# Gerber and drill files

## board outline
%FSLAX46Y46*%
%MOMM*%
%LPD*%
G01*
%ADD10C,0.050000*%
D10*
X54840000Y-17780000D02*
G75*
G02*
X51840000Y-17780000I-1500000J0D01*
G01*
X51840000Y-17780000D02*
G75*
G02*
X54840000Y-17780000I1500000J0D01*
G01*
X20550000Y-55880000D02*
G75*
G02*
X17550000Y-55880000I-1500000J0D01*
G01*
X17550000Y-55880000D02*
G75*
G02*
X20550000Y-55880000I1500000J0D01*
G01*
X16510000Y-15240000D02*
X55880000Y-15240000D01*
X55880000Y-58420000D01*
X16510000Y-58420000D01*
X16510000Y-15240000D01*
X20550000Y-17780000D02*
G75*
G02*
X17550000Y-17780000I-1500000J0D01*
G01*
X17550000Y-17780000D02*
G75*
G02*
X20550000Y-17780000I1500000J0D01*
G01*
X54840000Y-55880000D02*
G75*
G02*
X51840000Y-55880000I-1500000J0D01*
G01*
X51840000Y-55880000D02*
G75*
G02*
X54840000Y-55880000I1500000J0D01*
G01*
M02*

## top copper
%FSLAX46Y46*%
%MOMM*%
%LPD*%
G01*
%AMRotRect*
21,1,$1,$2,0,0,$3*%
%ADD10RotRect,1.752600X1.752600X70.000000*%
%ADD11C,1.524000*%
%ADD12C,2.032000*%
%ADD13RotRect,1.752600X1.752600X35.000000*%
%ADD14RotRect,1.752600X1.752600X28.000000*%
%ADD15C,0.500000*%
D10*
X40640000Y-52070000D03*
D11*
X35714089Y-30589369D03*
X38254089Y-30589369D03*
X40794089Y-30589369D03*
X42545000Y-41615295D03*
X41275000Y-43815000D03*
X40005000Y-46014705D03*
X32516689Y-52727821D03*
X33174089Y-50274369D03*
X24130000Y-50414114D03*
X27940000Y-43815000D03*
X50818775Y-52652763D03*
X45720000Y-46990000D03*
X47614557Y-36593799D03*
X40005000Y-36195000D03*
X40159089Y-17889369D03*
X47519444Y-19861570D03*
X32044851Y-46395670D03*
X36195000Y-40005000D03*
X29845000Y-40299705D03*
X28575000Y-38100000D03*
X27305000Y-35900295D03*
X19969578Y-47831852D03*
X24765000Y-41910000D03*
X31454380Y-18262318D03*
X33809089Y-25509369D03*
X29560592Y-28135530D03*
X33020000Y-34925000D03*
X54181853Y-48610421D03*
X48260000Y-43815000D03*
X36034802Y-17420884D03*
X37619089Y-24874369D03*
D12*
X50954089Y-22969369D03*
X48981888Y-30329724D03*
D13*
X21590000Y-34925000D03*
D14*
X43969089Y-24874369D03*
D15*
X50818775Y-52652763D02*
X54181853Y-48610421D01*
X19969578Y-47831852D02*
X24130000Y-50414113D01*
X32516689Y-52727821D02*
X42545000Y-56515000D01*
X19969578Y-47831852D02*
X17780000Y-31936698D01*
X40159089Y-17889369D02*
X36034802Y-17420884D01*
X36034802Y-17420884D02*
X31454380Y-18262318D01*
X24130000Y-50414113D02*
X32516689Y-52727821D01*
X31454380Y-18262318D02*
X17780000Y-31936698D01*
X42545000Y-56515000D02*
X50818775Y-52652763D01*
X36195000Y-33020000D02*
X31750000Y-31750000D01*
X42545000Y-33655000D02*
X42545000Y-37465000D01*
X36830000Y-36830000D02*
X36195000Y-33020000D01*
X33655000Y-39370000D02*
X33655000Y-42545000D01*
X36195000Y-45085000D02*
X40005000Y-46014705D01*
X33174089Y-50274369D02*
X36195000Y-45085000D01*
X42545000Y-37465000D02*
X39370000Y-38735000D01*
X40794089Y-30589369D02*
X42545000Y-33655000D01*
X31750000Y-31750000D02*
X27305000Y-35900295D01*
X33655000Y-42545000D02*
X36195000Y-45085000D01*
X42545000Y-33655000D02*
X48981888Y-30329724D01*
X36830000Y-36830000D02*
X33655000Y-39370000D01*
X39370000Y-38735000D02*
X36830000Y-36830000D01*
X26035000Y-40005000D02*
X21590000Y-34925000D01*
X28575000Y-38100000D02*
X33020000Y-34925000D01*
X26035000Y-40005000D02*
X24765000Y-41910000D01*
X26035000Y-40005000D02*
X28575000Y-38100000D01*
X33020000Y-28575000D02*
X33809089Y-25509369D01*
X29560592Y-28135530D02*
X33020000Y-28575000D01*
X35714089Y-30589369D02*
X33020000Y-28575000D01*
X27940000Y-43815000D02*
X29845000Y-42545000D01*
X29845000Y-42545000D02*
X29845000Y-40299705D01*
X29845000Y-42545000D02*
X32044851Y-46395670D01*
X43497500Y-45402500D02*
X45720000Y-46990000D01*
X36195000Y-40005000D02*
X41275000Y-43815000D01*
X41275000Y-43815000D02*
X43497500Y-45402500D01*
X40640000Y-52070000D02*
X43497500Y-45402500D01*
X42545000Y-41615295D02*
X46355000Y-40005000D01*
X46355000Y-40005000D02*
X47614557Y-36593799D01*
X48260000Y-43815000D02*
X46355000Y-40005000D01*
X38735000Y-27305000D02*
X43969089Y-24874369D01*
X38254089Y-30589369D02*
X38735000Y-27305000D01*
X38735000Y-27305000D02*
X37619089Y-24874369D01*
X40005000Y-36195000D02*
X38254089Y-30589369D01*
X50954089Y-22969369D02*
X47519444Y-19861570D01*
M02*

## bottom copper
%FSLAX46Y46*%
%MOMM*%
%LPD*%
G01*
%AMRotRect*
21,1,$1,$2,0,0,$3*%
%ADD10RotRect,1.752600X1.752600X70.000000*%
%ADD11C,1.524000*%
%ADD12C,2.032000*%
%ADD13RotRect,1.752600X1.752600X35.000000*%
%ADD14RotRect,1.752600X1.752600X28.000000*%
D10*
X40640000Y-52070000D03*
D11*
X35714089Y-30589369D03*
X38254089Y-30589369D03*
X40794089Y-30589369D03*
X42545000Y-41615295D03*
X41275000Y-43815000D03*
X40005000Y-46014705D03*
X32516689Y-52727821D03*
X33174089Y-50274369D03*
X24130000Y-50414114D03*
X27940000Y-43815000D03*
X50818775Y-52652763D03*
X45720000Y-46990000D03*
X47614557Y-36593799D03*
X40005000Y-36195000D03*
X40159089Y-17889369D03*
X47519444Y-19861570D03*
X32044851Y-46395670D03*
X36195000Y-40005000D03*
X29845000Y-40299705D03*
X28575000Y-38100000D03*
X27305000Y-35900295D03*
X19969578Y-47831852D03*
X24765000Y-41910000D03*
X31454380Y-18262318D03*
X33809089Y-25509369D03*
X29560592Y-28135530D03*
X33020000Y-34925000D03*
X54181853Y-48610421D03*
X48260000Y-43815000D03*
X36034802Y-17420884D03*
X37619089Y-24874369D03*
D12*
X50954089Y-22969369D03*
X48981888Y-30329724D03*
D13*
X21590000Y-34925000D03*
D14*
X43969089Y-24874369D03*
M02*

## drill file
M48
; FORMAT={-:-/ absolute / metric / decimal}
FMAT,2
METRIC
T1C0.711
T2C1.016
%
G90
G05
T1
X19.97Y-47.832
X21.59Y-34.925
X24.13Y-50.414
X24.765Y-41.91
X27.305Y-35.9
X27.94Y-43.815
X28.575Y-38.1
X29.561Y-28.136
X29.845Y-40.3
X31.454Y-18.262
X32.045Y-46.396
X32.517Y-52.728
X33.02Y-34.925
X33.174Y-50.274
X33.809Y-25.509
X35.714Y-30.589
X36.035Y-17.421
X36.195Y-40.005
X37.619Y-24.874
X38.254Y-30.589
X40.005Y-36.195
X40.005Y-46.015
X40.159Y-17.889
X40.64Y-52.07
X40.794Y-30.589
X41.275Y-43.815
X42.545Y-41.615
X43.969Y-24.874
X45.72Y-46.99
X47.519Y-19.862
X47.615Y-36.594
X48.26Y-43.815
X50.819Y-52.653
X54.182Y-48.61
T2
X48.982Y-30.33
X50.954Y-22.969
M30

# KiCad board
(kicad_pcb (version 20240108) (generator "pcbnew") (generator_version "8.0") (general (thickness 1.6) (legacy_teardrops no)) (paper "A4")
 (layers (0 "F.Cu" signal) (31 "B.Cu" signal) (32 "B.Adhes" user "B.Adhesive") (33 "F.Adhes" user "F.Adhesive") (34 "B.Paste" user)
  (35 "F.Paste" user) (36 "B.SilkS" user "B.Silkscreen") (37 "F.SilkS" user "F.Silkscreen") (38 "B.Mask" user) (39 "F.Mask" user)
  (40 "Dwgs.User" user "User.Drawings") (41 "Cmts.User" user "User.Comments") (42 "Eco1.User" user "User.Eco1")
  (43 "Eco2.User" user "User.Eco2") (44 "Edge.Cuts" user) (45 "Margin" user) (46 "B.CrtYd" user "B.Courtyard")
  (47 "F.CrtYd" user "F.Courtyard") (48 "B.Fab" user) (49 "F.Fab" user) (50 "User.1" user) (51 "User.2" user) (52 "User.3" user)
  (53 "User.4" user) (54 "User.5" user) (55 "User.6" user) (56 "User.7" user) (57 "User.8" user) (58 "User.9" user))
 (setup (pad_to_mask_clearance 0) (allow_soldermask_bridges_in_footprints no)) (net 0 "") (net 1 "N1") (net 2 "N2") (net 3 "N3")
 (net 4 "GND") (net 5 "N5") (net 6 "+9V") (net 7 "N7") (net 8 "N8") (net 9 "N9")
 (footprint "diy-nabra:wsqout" (layer "F.Cu") (at 40.64 52.07 70)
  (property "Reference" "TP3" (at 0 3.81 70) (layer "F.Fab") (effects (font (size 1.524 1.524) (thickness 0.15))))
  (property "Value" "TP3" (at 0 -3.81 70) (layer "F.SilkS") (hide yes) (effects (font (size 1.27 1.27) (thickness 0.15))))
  (pad "1" thru_hole rect (at 0 0 70) (size 1.7526 1.7526) (drill 0.7112) (layers "*.Cu" "*.Mask") (remove_unused_layers no) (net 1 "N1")))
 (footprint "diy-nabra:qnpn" (layer "F.Cu") (at 38.254089 30.589369 180)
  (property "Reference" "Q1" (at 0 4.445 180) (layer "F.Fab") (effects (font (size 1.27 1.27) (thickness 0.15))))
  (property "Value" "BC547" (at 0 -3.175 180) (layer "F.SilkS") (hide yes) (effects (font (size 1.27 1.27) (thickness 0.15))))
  (pad "1" thru_hole circle (at 2.54 0 180) (size 1.524 1.524) (drill 0.7112) (layers "*.Cu" "*.Mask") (remove_unused_layers no)
   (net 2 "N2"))
  (pad "2" thru_hole circle (at 0 0 180) (size 1.524 1.524) (drill 0.7112) (layers "*.Cu" "*.Mask") (remove_unused_layers no) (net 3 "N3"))
  (pad "3" thru_hole circle (at -2.54 0 180) (size 1.524 1.524) (drill 0.7112) (layers "*.Cu" "*.Mask") (remove_unused_layers no)
   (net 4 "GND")))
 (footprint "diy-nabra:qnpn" (layer "F.Cu") (at 41.275 43.815 60)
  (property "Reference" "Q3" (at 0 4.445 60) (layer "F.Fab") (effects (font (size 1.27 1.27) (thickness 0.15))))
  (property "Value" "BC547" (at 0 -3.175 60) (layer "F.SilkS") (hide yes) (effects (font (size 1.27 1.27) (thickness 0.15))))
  (pad "1" thru_hole circle (at 2.54 0 60) (size 1.524 1.524) (drill 0.7112) (layers "*.Cu" "*.Mask") (remove_unused_layers no) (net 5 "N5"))
  (pad "2" thru_hole circle (at 0 0 60) (size 1.524 1.524) (drill 0.7112) (layers "*.Cu" "*.Mask") (remove_unused_layers no) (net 1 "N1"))
  (pad "3" thru_hole circle (at -2.54 0 60) (size 1.524 1.524) (drill 0.7112) (layers "*.Cu" "*.Mask") (remove_unused_layers no)
   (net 4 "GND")))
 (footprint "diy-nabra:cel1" (layer "F.Cu") (at 33.174089 50.274369 -105)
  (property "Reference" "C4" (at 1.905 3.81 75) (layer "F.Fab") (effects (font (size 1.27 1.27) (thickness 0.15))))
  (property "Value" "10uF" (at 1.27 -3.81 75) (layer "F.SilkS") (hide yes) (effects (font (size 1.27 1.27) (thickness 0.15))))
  (pad "1" thru_hole circle (at 2.54 0 255) (size 1.524 1.524) (drill 0.7112) (layers "*.Cu" "*.Mask") (remove_unused_layers no)
   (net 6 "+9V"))
  (pad "2" thru_hole circle (at 0 0 255) (size 1.524 1.524) (drill 0.7112) (layers "*.Cu" "*.Mask") (remove_unused_layers no) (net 4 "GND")))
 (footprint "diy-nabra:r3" (layer "F.Cu") (at 27.94 43.815 -120)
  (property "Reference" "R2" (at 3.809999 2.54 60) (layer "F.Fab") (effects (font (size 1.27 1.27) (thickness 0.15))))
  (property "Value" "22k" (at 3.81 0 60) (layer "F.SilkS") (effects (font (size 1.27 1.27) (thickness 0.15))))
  (pad "1" thru_hole circle (at 7.62 0 240) (size 1.524 1.524) (drill 0.7112) (layers "*.Cu" "*.Mask") (remove_unused_layers no)
   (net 6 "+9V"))
  (pad "2" thru_hole circle (at 0 0 240) (size 1.524 1.524) (drill 0.7112) (layers "*.Cu" "*.Mask") (remove_unused_layers no) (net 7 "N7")))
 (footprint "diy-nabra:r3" (layer "F.Cu") (at 45.72 46.99 -48)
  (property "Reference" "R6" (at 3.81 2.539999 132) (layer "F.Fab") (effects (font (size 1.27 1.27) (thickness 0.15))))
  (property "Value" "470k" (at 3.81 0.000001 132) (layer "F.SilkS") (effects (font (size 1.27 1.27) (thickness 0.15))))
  (pad "1" thru_hole circle (at 7.619999 0 312) (size 1.524 1.524) (drill 0.7112) (layers "*.Cu" "*.Mask") (remove_unused_layers no)
   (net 6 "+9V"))
  (pad "2" thru_hole circle (at 0 0 312) (size 1.524 1.524) (drill 0.7112) (layers "*.Cu" "*.Mask") (remove_unused_layers no) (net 1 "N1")))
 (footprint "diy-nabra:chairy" (layer "F.Cu") (at 40.005 36.195 -3)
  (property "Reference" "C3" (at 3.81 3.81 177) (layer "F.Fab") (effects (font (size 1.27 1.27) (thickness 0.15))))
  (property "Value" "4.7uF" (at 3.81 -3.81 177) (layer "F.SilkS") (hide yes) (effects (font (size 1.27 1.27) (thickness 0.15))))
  (pad "1" thru_hole circle (at 7.62 -0.000001 357) (size 1.524 1.524) (drill 0.7112) (layers "*.Cu" "*.Mask") (remove_unused_layers no)
   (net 5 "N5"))
  (pad "2" thru_hole circle (at 0 0 357) (size 1.524 1.524) (drill 0.7112) (layers "*.Cu" "*.Mask") (remove_unused_layers no) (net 3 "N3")))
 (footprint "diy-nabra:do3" (layer "F.Cu") (at 40.159089 17.889369 -15)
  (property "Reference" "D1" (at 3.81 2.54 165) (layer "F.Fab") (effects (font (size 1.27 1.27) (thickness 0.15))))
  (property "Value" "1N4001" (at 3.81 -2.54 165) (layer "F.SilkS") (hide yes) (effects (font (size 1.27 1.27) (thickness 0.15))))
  (pad "1" thru_hole circle (at 0 0 345) (size 1.524 1.524) (drill 0.7112) (layers "*.Cu" "*.Mask") (remove_unused_layers no) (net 6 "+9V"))
  (pad "2" thru_hole circle (at 7.62 0 345) (size 1.524 1.524) (drill 0.7112) (layers "*.Cu" "*.Mask") (remove_unused_layers no)
   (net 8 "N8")))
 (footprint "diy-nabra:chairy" (layer "F.Cu") (at 36.195 40.005 -123)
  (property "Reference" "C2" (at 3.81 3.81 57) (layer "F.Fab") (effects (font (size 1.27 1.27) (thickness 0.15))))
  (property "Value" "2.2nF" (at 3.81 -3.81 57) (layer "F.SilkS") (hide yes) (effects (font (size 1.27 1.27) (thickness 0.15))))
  (pad "1" thru_hole circle (at 7.62 -0.000001 237) (size 1.524 1.524) (drill 0.7112) (layers "*.Cu" "*.Mask") (remove_unused_layers no)
   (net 7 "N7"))
  (pad "2" thru_hole circle (at 0 0 237) (size 1.524 1.524) (drill 0.7112) (layers "*.Cu" "*.Mask") (remove_unused_layers no) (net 1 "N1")))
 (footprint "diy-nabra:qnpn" (layer "F.Cu") (at 28.575 38.1 -60)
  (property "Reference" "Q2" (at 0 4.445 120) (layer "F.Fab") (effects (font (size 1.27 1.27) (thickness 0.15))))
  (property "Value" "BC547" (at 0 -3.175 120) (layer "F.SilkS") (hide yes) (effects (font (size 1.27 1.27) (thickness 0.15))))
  (pad "1" thru_hole circle (at 2.54 0 300) (size 1.524 1.524) (drill 0.7112) (layers "*.Cu" "*.Mask") (remove_unused_layers no)
   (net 7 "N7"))
  (pad "2" thru_hole circle (at 0 0 300) (size 1.524 1.524) (drill 0.7112) (layers "*.Cu" "*.Mask") (remove_unused_layers no) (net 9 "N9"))
  (pad "3" thru_hole circle (at -2.54 0 300) (size 1.524 1.524) (drill 0.7112) (layers "*.Cu" "*.Mask") (remove_unused_layers no)
   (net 4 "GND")))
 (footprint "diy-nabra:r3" (layer "F.Cu") (at 24.765 41.91 -129)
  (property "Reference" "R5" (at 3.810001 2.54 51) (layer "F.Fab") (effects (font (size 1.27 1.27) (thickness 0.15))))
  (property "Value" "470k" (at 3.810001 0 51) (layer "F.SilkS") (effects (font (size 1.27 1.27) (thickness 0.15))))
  (pad "1" thru_hole circle (at 7.62 0.000001 231) (size 1.524 1.524) (drill 0.7112) (layers "*.Cu" "*.Mask") (remove_unused_layers no)
   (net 6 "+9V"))
  (pad "2" thru_hole circle (at 0 0 231) (size 1.524 1.524) (drill 0.7112) (layers "*.Cu" "*.Mask") (remove_unused_layers no) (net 9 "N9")))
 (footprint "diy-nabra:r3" (layer "F.Cu") (at 33.809089 25.509369 108)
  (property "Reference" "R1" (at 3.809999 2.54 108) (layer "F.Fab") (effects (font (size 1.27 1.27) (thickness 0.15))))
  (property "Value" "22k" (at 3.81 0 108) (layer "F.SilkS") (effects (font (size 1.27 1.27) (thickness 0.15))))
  (pad "1" thru_hole circle (at 7.62 0.000001 108) (size 1.524 1.524) (drill 0.7112) (layers "*.Cu" "*.Mask") (remove_unused_layers no)
   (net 6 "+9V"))
  (pad "2" thru_hole circle (at 0 0 108) (size 1.524 1.524) (drill 0.7112) (layers "*.Cu" "*.Mask") (remove_unused_layers no) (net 2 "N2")))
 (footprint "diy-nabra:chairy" (layer "F.Cu") (at 33.02 34.925 117)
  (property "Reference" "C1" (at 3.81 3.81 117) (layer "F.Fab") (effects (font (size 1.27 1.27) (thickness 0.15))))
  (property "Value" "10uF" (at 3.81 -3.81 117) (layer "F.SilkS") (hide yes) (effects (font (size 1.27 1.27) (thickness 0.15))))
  (pad "1" thru_hole circle (at 7.62 0 117) (size 1.524 1.524) (drill 0.7112) (layers "*.Cu" "*.Mask") (remove_unused_layers no)
   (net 2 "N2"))
  (pad "2" thru_hole circle (at 0 0 117) (size 1.524 1.524) (drill 0.7112) (layers "*.Cu" "*.Mask") (remove_unused_layers no) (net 9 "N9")))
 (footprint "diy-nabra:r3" (layer "F.Cu") (at 48.26 43.815 -39)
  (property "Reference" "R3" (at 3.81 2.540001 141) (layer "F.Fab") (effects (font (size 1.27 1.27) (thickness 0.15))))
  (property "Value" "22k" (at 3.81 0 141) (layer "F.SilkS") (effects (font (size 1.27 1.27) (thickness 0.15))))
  (pad "1" thru_hole circle (at 7.62 -0.000001 321) (size 1.524 1.524) (drill 0.7112) (layers "*.Cu" "*.Mask") (remove_unused_layers no)
   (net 6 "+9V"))
  (pad "2" thru_hole circle (at 0 0 321) (size 1.524 1.524) (drill 0.7112) (layers "*.Cu" "*.Mask") (remove_unused_layers no) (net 5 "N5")))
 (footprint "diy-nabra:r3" (layer "F.Cu") (at 37.619089 24.874369 102)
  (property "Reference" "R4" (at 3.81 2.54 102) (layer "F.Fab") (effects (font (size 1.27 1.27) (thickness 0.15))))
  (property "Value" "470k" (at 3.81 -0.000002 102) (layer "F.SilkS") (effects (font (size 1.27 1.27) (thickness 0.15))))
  (pad "1" thru_hole circle (at 7.62 0 102) (size 1.524 1.524) (drill 0.7112) (layers "*.Cu" "*.Mask") (remove_unused_layers no)
   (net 6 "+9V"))
  (pad "2" thru_hole circle (at 0 0 102) (size 1.524 1.524) (drill 0.7112) (layers "*.Cu" "*.Mask") (remove_unused_layers no) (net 3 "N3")))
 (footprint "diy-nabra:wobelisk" (layer "F.Cu") (at 48.981888 30.329724 75)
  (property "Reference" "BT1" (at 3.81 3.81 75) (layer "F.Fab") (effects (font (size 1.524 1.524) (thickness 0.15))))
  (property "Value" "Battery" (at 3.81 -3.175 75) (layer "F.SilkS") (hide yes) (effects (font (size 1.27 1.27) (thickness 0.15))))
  (pad "1" thru_hole circle (at 7.62 0 75) (size 2.032 2.032) (drill 1.016) (layers "*.Cu" "*.Mask") (remove_unused_layers no) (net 8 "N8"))
  (pad "2" thru_hole circle (at 0 0 75) (size 2.032 2.032) (drill 1.016) (layers "*.Cu" "*.Mask") (remove_unused_layers no) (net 4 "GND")))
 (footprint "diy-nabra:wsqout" (layer "F.Cu") (at 21.59 34.925 35)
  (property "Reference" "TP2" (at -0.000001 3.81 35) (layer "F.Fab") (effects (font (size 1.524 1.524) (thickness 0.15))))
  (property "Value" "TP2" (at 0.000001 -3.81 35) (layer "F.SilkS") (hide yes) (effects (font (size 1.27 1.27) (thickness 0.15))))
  (pad "1" thru_hole rect (at 0 0 35) (size 1.7526 1.7526) (drill 0.7112) (layers "*.Cu" "*.Mask") (remove_unused_layers no) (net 9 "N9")))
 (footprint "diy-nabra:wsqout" (layer "F.Cu") (at 43.969089 24.874369 28)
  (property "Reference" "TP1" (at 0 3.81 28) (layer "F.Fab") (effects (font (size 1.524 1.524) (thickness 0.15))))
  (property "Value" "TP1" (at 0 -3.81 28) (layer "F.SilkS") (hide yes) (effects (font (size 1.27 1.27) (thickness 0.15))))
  (pad "1" thru_hole rect (at 0 0 28) (size 1.7526 1.7526) (drill 0.7112) (layers "*.Cu" "*.Mask") (remove_unused_layers no) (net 3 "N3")))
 (gr_circle (center 53.34 17.78) (end 54.84 17.78) (stroke (width 0.05) (type default)) (fill none) (layer "Edge.Cuts"))
 (gr_circle (center 19.05 55.88) (end 20.55 55.88) (stroke (width 0.05) (type default)) (fill none) (layer "Edge.Cuts"))
 (gr_rect (start 16.51 15.24) (end 55.88 58.42) (stroke (width 0.05) (type default)) (fill none) (layer "Edge.Cuts"))
 (gr_circle (center 19.05 17.78) (end 20.55 17.78) (stroke (width 0.05) (type default)) (fill none) (layer "Edge.Cuts"))
 (gr_circle (center 53.34 55.88) (end 54.84 55.88) (stroke (width 0.05) (type default)) (fill none) (layer "Edge.Cuts"))
 (segment (start 50.818775 52.652763) (end 54.181853 48.610421) (width 0.5) (layer "F.Cu") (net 6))
 (segment (start 19.969578 47.831852) (end 24.13 50.414113) (width 0.5) (layer "F.Cu") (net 6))
 (segment (start 32.516689 52.727821) (end 42.545 56.515) (width 0.5) (layer "F.Cu") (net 6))
 (segment (start 19.969578 47.831852) (end 17.78 31.936698) (width 0.5) (layer "F.Cu") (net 6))
 (segment (start 40.159089 17.889369) (end 36.034802 17.420884) (width 0.5) (layer "F.Cu") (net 6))
 (segment (start 36.034802 17.420884) (end 31.45438 18.262318) (width 0.5) (layer "F.Cu") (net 6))
 (segment (start 24.13 50.414113) (end 32.516689 52.727821) (width 0.5) (layer "F.Cu") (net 6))
 (segment (start 31.45438 18.262318) (end 17.78 31.936698) (width 0.5) (layer "F.Cu") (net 6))
 (segment (start 42.545 56.515) (end 50.818775 52.652763) (width 0.5) (layer "F.Cu") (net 6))
 (segment (start 36.195 33.02) (end 31.75 31.75) (width 0.5) (layer "F.Cu") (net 4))
 (segment (start 42.545 33.655) (end 42.545 37.465) (width 0.5) (layer "F.Cu") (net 4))
 (segment (start 36.83 36.83) (end 36.195 33.02) (width 0.5) (layer "F.Cu") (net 4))
 (segment (start 33.655 39.37) (end 33.655 42.545) (width 0.5) (layer "F.Cu") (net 4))
 (segment (start 36.195 45.085) (end 40.005 46.014705) (width 0.5) (layer "F.Cu") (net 4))
 (segment (start 33.174089 50.274369) (end 36.195 45.085) (width 0.5) (layer "F.Cu") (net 4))
 (segment (start 42.545 37.465) (end 39.37 38.735) (width 0.5) (layer "F.Cu") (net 4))
 (segment (start 40.794089 30.589369) (end 42.545 33.655) (width 0.5) (layer "F.Cu") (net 4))
 (segment (start 31.75 31.75) (end 27.305 35.900295) (width 0.5) (layer "F.Cu") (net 4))
 (segment (start 33.655 42.545) (end 36.195 45.085) (width 0.5) (layer "F.Cu") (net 4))
 (segment (start 42.545 33.655) (end 48.981888 30.329724) (width 0.5) (layer "F.Cu") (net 4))
 (segment (start 36.83 36.83) (end 33.655 39.37) (width 0.5) (layer "F.Cu") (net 4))
 (segment (start 39.37 38.735) (end 36.83 36.83) (width 0.5) (layer "F.Cu") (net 4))
 (segment (start 26.035 40.005) (end 21.59 34.925) (width 0.5) (layer "F.Cu") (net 9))
 (segment (start 28.575 38.1) (end 33.02 34.925) (width 0.5) (layer "F.Cu") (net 9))
 (segment (start 26.035 40.005) (end 24.765 41.91) (width 0.5) (layer "F.Cu") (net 9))
 (segment (start 26.035 40.005) (end 28.575 38.1) (width 0.5) (layer "F.Cu") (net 9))
 (segment (start 33.02 28.575) (end 33.809089 25.509369) (width 0.5) (layer "F.Cu") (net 2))
 (segment (start 29.560592 28.13553) (end 33.02 28.575) (width 0.5) (layer "F.Cu") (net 2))
 (segment (start 35.714089 30.589369) (end 33.02 28.575) (width 0.5) (layer "F.Cu") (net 2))
 (segment (start 27.94 43.815) (end 29.845 42.545) (width 0.5) (layer "F.Cu") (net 7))
 (segment (start 29.845 42.545) (end 29.845 40.299705) (width 0.5) (layer "F.Cu") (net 7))
 (segment (start 29.845 42.545) (end 32.044851 46.39567) (width 0.5) (layer "F.Cu") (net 7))
 (segment (start 43.4975 45.4025) (end 45.72 46.99) (width 0.5) (layer "F.Cu") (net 1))
 (segment (start 36.195 40.005) (end 41.275 43.815) (width 0.5) (layer "F.Cu") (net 1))
 (segment (start 41.275 43.815) (end 43.4975 45.4025) (width 0.5) (layer "F.Cu") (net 1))
 (segment (start 40.64 52.07) (end 43.4975 45.4025) (width 0.5) (layer "F.Cu") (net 1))
 (segment (start 42.545 41.615295) (end 46.355 40.005) (width 0.5) (layer "F.Cu") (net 5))
 (segment (start 46.355 40.005) (end 47.614557 36.593799) (width 0.5) (layer "F.Cu") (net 5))
 (segment (start 48.26 43.815) (end 46.355 40.005) (width 0.5) (layer "F.Cu") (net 5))
 (segment (start 38.735 27.305) (end 43.969089 24.874369) (width 0.5) (layer "F.Cu") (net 3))
 (segment (start 38.254089 30.589369) (end 38.735 27.305) (width 0.5) (layer "F.Cu") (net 3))
 (segment (start 38.735 27.305) (end 37.619089 24.874369) (width 0.5) (layer "F.Cu") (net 3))
 (segment (start 40.005 36.195) (end 38.254089 30.589369) (width 0.5) (layer "F.Cu") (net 3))
 (segment (start 50.954089 22.969369) (end 47.519444 19.86157) (width 0.5) (layer "F.Cu") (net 8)))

